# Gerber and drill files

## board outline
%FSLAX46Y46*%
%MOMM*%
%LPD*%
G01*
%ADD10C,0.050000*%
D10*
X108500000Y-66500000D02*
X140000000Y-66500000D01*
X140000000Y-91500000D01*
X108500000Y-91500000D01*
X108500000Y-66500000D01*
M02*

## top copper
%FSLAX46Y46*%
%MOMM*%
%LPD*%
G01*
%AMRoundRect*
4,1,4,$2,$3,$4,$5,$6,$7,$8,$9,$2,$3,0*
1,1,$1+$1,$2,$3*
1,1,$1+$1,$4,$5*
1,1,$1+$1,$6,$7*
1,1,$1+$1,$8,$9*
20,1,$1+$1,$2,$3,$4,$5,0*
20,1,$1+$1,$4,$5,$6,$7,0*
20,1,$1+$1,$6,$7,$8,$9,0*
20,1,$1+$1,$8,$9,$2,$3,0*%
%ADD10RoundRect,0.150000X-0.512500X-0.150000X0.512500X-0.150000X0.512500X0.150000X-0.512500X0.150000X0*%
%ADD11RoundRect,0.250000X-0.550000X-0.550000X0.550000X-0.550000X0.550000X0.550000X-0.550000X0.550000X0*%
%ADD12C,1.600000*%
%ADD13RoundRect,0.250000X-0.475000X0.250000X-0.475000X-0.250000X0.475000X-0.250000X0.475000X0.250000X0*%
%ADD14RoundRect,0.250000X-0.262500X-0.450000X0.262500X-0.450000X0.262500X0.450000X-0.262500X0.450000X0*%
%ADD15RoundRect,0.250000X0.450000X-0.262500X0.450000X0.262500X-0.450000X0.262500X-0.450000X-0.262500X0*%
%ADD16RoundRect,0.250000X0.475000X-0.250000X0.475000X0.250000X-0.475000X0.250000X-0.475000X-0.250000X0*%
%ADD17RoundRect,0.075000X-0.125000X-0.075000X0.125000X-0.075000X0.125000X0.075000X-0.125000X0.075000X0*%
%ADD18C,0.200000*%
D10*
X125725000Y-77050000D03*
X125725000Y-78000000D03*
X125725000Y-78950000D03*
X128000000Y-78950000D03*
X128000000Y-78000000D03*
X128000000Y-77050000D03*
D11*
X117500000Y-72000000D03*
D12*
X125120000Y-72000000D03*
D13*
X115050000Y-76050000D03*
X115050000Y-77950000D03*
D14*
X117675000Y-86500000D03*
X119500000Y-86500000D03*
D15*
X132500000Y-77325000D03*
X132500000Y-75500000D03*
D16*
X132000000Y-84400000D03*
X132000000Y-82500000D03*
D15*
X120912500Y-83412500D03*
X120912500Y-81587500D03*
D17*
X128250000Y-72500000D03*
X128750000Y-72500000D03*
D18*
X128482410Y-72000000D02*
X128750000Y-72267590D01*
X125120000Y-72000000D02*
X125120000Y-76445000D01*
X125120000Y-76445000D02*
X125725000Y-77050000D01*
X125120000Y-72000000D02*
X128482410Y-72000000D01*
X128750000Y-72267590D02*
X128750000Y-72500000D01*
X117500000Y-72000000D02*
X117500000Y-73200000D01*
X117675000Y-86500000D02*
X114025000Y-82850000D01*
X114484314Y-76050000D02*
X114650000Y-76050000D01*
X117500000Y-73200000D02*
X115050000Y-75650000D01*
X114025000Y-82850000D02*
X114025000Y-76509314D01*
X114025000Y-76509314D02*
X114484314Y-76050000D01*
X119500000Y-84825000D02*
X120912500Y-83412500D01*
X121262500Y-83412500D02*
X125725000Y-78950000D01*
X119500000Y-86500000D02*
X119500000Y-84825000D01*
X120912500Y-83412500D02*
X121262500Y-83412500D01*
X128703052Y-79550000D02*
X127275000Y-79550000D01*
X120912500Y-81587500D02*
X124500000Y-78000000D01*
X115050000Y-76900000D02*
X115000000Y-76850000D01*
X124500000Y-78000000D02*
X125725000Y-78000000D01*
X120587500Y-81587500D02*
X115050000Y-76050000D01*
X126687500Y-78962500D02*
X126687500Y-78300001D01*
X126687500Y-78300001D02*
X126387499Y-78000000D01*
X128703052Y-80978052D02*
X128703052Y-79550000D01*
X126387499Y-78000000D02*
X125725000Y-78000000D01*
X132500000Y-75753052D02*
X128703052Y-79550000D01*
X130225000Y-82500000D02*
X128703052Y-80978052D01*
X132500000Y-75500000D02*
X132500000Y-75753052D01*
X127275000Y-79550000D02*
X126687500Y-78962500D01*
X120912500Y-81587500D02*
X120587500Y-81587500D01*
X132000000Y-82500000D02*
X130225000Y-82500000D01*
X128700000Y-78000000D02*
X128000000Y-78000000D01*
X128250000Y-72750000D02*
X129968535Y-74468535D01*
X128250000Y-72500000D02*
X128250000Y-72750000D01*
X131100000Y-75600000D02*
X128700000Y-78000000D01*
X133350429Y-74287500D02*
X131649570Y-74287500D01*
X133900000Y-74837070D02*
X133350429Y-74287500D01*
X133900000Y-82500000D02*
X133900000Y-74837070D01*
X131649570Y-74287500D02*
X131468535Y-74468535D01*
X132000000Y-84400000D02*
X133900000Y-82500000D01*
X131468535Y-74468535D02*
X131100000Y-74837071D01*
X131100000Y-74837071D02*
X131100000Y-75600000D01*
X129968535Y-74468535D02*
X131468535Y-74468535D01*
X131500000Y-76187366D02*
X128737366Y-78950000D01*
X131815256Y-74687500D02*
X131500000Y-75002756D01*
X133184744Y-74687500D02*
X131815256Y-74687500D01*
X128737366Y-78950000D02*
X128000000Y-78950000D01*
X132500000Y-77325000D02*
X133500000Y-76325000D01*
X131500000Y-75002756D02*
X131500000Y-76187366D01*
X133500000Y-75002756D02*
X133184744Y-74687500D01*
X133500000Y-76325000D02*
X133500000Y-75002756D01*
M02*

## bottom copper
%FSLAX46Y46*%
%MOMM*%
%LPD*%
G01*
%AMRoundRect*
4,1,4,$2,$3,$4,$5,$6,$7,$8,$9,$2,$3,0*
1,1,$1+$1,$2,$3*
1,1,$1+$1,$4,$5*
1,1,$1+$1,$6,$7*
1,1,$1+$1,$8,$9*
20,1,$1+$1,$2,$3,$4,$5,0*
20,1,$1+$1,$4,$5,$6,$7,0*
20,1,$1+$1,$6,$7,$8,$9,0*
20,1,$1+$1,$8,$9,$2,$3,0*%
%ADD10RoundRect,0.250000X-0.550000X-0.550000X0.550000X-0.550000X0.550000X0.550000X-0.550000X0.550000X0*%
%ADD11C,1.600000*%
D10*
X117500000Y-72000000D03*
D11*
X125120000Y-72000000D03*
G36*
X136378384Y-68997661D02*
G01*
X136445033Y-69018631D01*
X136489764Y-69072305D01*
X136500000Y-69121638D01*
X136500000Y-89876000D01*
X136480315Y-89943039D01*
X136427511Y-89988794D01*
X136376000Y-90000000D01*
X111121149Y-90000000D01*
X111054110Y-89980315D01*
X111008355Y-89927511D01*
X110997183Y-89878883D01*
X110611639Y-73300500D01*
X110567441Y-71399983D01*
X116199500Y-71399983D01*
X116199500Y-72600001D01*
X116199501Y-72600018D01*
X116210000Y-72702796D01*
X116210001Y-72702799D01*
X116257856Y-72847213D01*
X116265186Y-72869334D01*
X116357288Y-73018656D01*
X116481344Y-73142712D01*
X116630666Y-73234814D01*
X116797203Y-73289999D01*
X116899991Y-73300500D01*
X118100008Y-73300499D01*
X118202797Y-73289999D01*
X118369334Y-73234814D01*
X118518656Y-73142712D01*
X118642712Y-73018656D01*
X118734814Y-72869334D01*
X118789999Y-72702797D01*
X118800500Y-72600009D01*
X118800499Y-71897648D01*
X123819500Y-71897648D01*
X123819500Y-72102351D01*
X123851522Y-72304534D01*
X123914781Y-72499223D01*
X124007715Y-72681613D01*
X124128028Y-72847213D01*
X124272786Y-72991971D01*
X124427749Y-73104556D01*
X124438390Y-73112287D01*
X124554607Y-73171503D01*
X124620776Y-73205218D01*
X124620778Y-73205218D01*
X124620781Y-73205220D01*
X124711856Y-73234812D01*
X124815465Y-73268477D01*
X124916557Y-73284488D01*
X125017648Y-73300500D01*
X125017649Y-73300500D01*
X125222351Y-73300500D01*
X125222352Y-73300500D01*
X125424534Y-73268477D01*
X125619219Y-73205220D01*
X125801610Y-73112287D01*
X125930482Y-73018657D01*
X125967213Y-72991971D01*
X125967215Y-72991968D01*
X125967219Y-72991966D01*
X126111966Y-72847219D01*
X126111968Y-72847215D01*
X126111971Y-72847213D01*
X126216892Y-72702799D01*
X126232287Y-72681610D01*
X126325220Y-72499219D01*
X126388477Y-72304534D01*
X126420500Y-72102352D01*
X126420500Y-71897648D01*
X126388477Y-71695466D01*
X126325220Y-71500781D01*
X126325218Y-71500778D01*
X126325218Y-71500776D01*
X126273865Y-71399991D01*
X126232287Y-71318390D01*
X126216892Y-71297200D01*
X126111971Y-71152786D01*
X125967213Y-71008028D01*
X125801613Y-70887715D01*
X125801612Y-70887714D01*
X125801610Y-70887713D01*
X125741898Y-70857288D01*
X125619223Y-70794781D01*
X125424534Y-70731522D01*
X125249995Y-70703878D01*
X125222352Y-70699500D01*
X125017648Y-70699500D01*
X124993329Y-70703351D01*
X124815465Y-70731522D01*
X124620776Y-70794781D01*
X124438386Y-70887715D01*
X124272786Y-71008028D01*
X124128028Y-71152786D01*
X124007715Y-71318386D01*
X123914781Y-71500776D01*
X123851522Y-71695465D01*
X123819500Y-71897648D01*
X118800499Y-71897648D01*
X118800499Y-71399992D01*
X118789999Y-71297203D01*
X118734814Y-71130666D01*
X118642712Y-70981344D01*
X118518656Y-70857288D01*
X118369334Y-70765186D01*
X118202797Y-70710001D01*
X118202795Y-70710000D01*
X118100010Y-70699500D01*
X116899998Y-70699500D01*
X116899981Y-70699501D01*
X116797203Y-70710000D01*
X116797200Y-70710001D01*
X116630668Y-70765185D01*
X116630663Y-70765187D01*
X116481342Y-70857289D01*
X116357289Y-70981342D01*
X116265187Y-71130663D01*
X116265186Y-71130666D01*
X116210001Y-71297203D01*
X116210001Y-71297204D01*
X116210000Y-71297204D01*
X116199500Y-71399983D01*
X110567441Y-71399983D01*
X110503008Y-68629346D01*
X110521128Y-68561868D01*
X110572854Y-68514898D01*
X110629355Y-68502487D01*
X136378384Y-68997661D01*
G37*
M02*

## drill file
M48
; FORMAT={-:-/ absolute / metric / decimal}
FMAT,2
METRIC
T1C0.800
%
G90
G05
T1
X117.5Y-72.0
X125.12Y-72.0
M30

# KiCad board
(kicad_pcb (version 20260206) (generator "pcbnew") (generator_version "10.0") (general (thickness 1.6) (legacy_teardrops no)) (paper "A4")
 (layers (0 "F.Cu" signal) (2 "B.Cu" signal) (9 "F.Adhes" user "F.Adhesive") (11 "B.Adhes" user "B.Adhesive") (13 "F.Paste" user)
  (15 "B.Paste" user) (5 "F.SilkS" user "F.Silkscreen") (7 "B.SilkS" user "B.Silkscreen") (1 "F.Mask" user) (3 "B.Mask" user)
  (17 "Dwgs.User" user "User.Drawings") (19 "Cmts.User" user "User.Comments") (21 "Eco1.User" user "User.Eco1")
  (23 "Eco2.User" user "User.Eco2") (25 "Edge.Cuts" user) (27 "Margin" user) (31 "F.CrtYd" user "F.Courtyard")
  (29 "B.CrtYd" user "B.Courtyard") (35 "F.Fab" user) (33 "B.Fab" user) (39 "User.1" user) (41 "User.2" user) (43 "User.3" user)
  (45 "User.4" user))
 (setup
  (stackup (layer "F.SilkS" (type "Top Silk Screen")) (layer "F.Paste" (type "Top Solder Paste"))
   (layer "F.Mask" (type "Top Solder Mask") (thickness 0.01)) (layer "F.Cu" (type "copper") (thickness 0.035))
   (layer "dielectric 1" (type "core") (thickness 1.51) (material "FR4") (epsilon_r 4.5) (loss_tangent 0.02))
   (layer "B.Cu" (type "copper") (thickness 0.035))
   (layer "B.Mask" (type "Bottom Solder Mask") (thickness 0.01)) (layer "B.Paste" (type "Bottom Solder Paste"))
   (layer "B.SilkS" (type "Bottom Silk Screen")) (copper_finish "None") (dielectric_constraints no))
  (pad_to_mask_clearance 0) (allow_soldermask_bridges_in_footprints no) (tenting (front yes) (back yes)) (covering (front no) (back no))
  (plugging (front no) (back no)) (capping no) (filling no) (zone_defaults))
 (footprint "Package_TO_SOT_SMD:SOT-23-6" (layer "F.Cu") (at 126.8625 78)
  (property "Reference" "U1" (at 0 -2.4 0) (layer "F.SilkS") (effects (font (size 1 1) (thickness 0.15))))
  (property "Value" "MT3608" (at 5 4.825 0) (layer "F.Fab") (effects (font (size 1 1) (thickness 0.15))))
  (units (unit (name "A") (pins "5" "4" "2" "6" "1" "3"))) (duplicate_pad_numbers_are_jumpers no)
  (pad "1" smd roundrect (at -1.1375 -0.95) (size 1.325 0.6) (layers "F.Cu" "F.Mask" "F.Paste") (roundrect_rratio 0.25) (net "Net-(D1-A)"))
  (pad "2" smd roundrect (at -1.1375 0) (size 1.325 0.6) (layers "F.Cu" "F.Mask" "F.Paste") (roundrect_rratio 0.25) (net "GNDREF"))
  (pad "3" smd roundrect (at -1.1375 0.95) (size 1.325 0.6) (layers "F.Cu" "F.Mask" "F.Paste") (roundrect_rratio 0.25) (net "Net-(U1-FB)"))
  (pad "4" smd roundrect (at 1.1375 0.95) (size 1.325 0.6) (layers "F.Cu" "F.Mask" "F.Paste") (roundrect_rratio 0.25) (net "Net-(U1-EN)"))
  (pad "5" smd roundrect (at 1.1375 0) (size 1.325 0.6) (layers "F.Cu" "F.Mask" "F.Paste") (roundrect_rratio 0.25) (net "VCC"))
  (pad "6" smd roundrect (at 1.1375 -0.95) (size 1.325 0.6) (layers "F.Cu" "F.Mask" "F.Paste") (roundrect_rratio 0.25)
   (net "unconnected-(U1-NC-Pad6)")))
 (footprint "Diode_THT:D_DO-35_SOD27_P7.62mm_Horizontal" (layer "F.Cu") (at 117.5 72)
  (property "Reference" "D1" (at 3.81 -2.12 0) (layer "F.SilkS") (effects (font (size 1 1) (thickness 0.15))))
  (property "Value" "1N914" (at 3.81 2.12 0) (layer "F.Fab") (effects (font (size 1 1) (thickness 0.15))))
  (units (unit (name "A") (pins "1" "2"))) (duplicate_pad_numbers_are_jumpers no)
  (pad "1" thru_hole roundrect (at 0 0) (size 1.6 1.6) (drill 0.8) (layers "*.Cu" "*.Mask") (remove_unused_layers no)
   (roundrect_rratio 0.15625) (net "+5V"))
  (pad "2" thru_hole circle (at 7.62 0) (size 1.6 1.6) (drill 0.8) (layers "*.Cu" "*.Mask") (remove_unused_layers no) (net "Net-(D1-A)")))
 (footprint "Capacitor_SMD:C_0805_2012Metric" (layer "F.Cu") (at 115.05 77 -90)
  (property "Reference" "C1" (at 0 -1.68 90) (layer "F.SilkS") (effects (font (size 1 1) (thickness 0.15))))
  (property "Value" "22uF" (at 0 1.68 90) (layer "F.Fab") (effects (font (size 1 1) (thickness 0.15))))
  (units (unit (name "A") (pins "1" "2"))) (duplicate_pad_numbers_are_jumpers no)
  (pad "1" smd roundrect (at -0.95 0 270) (size 1 1.45) (layers "F.Cu" "F.Mask" "F.Paste") (roundrect_rratio 0.25) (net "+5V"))
  (pad "2" smd roundrect (at 0.95 0 270) (size 1 1.45) (layers "F.Cu" "F.Mask" "F.Paste") (roundrect_rratio 0.25) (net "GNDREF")))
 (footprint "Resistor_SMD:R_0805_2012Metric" (layer "F.Cu") (at 118.5875 86.5)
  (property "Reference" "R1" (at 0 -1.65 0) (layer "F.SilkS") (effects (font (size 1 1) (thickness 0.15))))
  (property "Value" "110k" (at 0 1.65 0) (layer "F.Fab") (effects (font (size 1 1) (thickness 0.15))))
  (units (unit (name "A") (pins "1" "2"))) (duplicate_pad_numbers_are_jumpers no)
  (pad "1" smd roundrect (at -0.9125 0) (size 1.025 1.4) (layers "F.Cu" "F.Mask" "F.Paste") (roundrect_rratio 0.243902) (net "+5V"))
  (pad "2" smd roundrect (at 0.9125 0) (size 1.025 1.4) (layers "F.Cu" "F.Mask" "F.Paste") (roundrect_rratio 0.243902) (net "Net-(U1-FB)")))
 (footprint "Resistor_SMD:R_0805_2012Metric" (layer "F.Cu") (at 132.5 76.4125 90)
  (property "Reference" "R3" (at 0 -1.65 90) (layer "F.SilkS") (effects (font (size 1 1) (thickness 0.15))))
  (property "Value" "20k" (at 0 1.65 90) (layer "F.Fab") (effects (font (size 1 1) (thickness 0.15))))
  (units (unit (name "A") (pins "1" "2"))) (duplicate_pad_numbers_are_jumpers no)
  (pad "1" smd roundrect (at -0.9125 0 90) (size 1.025 1.4) (layers "F.Cu" "F.Mask" "F.Paste") (roundrect_rratio 0.243902)
   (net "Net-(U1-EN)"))
  (pad "2" smd roundrect (at 0.9125 0 90) (size 1.025 1.4) (layers "F.Cu" "F.Mask" "F.Paste") (roundrect_rratio 0.243902) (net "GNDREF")))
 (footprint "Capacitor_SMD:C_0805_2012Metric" (layer "F.Cu") (at 132 83.45 90)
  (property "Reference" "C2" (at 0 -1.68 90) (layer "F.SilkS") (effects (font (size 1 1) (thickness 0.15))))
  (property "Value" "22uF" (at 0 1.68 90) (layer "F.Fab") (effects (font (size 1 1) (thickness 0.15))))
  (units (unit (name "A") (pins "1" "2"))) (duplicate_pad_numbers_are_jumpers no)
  (pad "1" smd roundrect (at -0.95 0 90) (size 1 1.45) (layers "F.Cu" "F.Mask" "F.Paste") (roundrect_rratio 0.25) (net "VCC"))
  (pad "2" smd roundrect (at 0.95 0 90) (size 1 1.45) (layers "F.Cu" "F.Mask" "F.Paste") (roundrect_rratio 0.25) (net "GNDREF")))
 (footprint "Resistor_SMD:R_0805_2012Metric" (layer "F.Cu") (at 120.9125 82.5 90)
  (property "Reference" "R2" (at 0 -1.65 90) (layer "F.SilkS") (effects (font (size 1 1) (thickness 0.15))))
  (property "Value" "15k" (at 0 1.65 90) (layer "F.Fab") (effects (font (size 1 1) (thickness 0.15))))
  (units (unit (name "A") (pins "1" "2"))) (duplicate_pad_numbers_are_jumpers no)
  (pad "1" smd roundrect (at -0.9125 0 90) (size 1.025 1.4) (layers "F.Cu" "F.Mask" "F.Paste") (roundrect_rratio 0.243902)
   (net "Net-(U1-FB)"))
  (pad "2" smd roundrect (at 0.9125 0 90) (size 1.025 1.4) (layers "F.Cu" "F.Mask" "F.Paste") (roundrect_rratio 0.243902) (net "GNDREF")))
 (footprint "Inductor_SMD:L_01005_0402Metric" (layer "F.Cu") (at 128.5 72.5)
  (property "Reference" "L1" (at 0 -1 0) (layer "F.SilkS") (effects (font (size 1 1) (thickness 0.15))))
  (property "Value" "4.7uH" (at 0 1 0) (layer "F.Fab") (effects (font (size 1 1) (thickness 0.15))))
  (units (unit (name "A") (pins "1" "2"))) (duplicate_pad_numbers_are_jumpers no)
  (pad "" smd roundrect (at -0.275 0) (size 0.27 0.27) (layers "F.Paste") (roundrect_rratio 0.25))
  (pad "" smd roundrect (at 0.275 0) (size 0.27 0.27) (layers "F.Paste") (roundrect_rratio 0.25))
  (pad "1" smd roundrect (at -0.25 0) (size 0.4 0.3) (layers "F.Cu" "F.Mask") (roundrect_rratio 0.25) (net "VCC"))
  (pad "2" smd roundrect (at 0.25 0) (size 0.4 0.3) (layers "F.Cu" "F.Mask") (roundrect_rratio 0.25) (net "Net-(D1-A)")))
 (gr_rect (start 108.5 66.5) (end 140 91.5) (stroke (width 0.05) (type default)) (fill no) (layer "Edge.Cuts"))
 (segment (start 128.48241 72) (end 128.75 72.26759) (width 0.2) (layer "F.Cu") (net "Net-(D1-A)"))
 (segment (start 125.12 72) (end 125.12 76.445) (width 0.2) (layer "F.Cu") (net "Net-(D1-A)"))
 (segment (start 125.12 76.445) (end 125.725 77.05) (width 0.2) (layer "F.Cu") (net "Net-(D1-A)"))
 (segment (start 125.12 72) (end 128.48241 72) (width 0.2) (layer "F.Cu") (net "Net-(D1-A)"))
 (segment (start 128.75 72.26759) (end 128.75 72.5) (width 0.2) (layer "F.Cu") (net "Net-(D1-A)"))
 (segment (start 117.5 72) (end 117.5 73.2) (width 0.2) (layer "F.Cu") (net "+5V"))
 (segment (start 117.675 86.5) (end 114.025 82.85) (width 0.2) (layer "F.Cu") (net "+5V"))
 (segment (start 114.484314 76.05) (end 114.65 76.05) (width 0.2) (layer "F.Cu") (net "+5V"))
 (segment (start 117.5 73.2) (end 115.05 75.65) (width 0.2) (layer "F.Cu") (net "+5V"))
 (segment (start 114.025 82.85) (end 114.025 76.509314) (width 0.2) (layer "F.Cu") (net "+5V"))
 (segment (start 114.025 76.509314) (end 114.484314 76.05) (width 0.2) (layer "F.Cu") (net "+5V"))
 (segment (start 119.5 84.825) (end 120.9125 83.4125) (width 0.2) (layer "F.Cu") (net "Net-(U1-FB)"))
 (segment (start 121.2625 83.4125) (end 125.725 78.95) (width 0.2) (layer "F.Cu") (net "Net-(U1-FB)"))
 (segment (start 119.5 86.5) (end 119.5 84.825) (width 0.2) (layer "F.Cu") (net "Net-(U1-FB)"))
 (segment (start 120.9125 83.4125) (end 121.2625 83.4125) (width 0.2) (layer "F.Cu") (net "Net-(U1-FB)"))
 (segment (start 128.703052 79.55) (end 127.275 79.55) (width 0.2) (layer "F.Cu") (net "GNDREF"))
 (segment (start 120.9125 81.5875) (end 124.5 78) (width 0.2) (layer "F.Cu") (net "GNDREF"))
 (segment (start 115.05 76.9) (end 115 76.85) (width 0.2) (layer "F.Cu") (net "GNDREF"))
 (segment (start 124.5 78) (end 125.725 78) (width 0.2) (layer "F.Cu") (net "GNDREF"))
 (segment (start 120.5875 81.5875) (end 115.05 76.05) (width 0.2) (layer "F.Cu") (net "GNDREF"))
 (segment (start 126.6875 78.9625) (end 126.6875 78.300001) (width 0.2) (layer "F.Cu") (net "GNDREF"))
 (segment (start 126.6875 78.300001) (end 126.387499 78) (width 0.2) (layer "F.Cu") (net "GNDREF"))
 (segment (start 128.703052 80.978052) (end 128.703052 79.55) (width 0.2) (layer "F.Cu") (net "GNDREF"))
 (segment (start 126.387499 78) (end 125.725 78) (width 0.2) (layer "F.Cu") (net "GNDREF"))
 (segment (start 132.5 75.753052) (end 128.703052 79.55) (width 0.2) (layer "F.Cu") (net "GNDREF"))
 (segment (start 130.225 82.5) (end 128.703052 80.978052) (width 0.2) (layer "F.Cu") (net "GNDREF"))
 (segment (start 132.5 75.5) (end 132.5 75.753052) (width 0.2) (layer "F.Cu") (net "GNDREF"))
 (segment (start 127.275 79.55) (end 126.6875 78.9625) (width 0.2) (layer "F.Cu") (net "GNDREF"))
 (segment (start 120.9125 81.5875) (end 120.5875 81.5875) (width 0.2) (layer "F.Cu") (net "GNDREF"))
 (segment (start 132 82.5) (end 130.225 82.5) (width 0.2) (layer "F.Cu") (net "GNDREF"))
 (segment (start 128.7 78) (end 128 78) (width 0.2) (layer "F.Cu") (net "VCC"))
 (segment (start 128.25 72.75) (end 129.968535 74.468535) (width 0.2) (layer "F.Cu") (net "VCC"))
 (segment (start 128.25 72.5) (end 128.25 72.75) (width 0.2) (layer "F.Cu") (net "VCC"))
 (segment (start 131.1 75.6) (end 128.7 78) (width 0.2) (layer "F.Cu") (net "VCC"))
 (segment (start 133.350429 74.2875) (end 131.64957 74.2875) (width 0.2) (layer "F.Cu") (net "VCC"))
 (segment (start 133.9 74.83707) (end 133.350429 74.2875) (width 0.2) (layer "F.Cu") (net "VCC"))
 (segment (start 133.9 82.5) (end 133.9 74.83707) (width 0.2) (layer "F.Cu") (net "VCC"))
 (segment (start 131.64957 74.2875) (end 131.468535 74.468535) (width 0.2) (layer "F.Cu") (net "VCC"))
 (segment (start 132 84.4) (end 133.9 82.5) (width 0.2) (layer "F.Cu") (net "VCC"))
 (segment (start 131.468535 74.468535) (end 131.1 74.837071) (width 0.2) (layer "F.Cu") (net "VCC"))
 (segment (start 131.1 74.837071) (end 131.1 75.6) (width 0.2) (layer "F.Cu") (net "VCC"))
 (segment (start 129.968535 74.468535) (end 131.468535 74.468535) (width 0.2) (layer "F.Cu") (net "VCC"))
 (segment (start 131.5 76.187366) (end 128.737366 78.95) (width 0.2) (layer "F.Cu") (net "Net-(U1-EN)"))
 (segment (start 131.815256 74.6875) (end 131.5 75.002756) (width 0.2) (layer "F.Cu") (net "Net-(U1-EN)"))
 (segment (start 133.184744 74.6875) (end 131.815256 74.6875) (width 0.2) (layer "F.Cu") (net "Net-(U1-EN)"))
 (segment (start 128.737366 78.95) (end 128 78.95) (width 0.2) (layer "F.Cu") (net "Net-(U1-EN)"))
 (segment (start 132.5 77.325) (end 133.5 76.325) (width 0.2) (layer "F.Cu") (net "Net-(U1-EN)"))
 (segment (start 131.5 75.002756) (end 131.5 76.187366) (width 0.2) (layer "F.Cu") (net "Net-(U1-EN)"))
 (segment (start 133.5 75.002756) (end 133.184744 74.6875) (width 0.2) (layer "F.Cu") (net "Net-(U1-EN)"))
 (segment (start 133.5 76.325) (end 133.5 75.002756) (width 0.2) (layer "F.Cu") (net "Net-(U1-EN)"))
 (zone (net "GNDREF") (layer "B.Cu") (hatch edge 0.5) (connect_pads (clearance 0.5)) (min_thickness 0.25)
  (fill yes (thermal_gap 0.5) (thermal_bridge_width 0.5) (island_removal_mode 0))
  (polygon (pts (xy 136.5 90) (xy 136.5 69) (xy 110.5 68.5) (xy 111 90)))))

